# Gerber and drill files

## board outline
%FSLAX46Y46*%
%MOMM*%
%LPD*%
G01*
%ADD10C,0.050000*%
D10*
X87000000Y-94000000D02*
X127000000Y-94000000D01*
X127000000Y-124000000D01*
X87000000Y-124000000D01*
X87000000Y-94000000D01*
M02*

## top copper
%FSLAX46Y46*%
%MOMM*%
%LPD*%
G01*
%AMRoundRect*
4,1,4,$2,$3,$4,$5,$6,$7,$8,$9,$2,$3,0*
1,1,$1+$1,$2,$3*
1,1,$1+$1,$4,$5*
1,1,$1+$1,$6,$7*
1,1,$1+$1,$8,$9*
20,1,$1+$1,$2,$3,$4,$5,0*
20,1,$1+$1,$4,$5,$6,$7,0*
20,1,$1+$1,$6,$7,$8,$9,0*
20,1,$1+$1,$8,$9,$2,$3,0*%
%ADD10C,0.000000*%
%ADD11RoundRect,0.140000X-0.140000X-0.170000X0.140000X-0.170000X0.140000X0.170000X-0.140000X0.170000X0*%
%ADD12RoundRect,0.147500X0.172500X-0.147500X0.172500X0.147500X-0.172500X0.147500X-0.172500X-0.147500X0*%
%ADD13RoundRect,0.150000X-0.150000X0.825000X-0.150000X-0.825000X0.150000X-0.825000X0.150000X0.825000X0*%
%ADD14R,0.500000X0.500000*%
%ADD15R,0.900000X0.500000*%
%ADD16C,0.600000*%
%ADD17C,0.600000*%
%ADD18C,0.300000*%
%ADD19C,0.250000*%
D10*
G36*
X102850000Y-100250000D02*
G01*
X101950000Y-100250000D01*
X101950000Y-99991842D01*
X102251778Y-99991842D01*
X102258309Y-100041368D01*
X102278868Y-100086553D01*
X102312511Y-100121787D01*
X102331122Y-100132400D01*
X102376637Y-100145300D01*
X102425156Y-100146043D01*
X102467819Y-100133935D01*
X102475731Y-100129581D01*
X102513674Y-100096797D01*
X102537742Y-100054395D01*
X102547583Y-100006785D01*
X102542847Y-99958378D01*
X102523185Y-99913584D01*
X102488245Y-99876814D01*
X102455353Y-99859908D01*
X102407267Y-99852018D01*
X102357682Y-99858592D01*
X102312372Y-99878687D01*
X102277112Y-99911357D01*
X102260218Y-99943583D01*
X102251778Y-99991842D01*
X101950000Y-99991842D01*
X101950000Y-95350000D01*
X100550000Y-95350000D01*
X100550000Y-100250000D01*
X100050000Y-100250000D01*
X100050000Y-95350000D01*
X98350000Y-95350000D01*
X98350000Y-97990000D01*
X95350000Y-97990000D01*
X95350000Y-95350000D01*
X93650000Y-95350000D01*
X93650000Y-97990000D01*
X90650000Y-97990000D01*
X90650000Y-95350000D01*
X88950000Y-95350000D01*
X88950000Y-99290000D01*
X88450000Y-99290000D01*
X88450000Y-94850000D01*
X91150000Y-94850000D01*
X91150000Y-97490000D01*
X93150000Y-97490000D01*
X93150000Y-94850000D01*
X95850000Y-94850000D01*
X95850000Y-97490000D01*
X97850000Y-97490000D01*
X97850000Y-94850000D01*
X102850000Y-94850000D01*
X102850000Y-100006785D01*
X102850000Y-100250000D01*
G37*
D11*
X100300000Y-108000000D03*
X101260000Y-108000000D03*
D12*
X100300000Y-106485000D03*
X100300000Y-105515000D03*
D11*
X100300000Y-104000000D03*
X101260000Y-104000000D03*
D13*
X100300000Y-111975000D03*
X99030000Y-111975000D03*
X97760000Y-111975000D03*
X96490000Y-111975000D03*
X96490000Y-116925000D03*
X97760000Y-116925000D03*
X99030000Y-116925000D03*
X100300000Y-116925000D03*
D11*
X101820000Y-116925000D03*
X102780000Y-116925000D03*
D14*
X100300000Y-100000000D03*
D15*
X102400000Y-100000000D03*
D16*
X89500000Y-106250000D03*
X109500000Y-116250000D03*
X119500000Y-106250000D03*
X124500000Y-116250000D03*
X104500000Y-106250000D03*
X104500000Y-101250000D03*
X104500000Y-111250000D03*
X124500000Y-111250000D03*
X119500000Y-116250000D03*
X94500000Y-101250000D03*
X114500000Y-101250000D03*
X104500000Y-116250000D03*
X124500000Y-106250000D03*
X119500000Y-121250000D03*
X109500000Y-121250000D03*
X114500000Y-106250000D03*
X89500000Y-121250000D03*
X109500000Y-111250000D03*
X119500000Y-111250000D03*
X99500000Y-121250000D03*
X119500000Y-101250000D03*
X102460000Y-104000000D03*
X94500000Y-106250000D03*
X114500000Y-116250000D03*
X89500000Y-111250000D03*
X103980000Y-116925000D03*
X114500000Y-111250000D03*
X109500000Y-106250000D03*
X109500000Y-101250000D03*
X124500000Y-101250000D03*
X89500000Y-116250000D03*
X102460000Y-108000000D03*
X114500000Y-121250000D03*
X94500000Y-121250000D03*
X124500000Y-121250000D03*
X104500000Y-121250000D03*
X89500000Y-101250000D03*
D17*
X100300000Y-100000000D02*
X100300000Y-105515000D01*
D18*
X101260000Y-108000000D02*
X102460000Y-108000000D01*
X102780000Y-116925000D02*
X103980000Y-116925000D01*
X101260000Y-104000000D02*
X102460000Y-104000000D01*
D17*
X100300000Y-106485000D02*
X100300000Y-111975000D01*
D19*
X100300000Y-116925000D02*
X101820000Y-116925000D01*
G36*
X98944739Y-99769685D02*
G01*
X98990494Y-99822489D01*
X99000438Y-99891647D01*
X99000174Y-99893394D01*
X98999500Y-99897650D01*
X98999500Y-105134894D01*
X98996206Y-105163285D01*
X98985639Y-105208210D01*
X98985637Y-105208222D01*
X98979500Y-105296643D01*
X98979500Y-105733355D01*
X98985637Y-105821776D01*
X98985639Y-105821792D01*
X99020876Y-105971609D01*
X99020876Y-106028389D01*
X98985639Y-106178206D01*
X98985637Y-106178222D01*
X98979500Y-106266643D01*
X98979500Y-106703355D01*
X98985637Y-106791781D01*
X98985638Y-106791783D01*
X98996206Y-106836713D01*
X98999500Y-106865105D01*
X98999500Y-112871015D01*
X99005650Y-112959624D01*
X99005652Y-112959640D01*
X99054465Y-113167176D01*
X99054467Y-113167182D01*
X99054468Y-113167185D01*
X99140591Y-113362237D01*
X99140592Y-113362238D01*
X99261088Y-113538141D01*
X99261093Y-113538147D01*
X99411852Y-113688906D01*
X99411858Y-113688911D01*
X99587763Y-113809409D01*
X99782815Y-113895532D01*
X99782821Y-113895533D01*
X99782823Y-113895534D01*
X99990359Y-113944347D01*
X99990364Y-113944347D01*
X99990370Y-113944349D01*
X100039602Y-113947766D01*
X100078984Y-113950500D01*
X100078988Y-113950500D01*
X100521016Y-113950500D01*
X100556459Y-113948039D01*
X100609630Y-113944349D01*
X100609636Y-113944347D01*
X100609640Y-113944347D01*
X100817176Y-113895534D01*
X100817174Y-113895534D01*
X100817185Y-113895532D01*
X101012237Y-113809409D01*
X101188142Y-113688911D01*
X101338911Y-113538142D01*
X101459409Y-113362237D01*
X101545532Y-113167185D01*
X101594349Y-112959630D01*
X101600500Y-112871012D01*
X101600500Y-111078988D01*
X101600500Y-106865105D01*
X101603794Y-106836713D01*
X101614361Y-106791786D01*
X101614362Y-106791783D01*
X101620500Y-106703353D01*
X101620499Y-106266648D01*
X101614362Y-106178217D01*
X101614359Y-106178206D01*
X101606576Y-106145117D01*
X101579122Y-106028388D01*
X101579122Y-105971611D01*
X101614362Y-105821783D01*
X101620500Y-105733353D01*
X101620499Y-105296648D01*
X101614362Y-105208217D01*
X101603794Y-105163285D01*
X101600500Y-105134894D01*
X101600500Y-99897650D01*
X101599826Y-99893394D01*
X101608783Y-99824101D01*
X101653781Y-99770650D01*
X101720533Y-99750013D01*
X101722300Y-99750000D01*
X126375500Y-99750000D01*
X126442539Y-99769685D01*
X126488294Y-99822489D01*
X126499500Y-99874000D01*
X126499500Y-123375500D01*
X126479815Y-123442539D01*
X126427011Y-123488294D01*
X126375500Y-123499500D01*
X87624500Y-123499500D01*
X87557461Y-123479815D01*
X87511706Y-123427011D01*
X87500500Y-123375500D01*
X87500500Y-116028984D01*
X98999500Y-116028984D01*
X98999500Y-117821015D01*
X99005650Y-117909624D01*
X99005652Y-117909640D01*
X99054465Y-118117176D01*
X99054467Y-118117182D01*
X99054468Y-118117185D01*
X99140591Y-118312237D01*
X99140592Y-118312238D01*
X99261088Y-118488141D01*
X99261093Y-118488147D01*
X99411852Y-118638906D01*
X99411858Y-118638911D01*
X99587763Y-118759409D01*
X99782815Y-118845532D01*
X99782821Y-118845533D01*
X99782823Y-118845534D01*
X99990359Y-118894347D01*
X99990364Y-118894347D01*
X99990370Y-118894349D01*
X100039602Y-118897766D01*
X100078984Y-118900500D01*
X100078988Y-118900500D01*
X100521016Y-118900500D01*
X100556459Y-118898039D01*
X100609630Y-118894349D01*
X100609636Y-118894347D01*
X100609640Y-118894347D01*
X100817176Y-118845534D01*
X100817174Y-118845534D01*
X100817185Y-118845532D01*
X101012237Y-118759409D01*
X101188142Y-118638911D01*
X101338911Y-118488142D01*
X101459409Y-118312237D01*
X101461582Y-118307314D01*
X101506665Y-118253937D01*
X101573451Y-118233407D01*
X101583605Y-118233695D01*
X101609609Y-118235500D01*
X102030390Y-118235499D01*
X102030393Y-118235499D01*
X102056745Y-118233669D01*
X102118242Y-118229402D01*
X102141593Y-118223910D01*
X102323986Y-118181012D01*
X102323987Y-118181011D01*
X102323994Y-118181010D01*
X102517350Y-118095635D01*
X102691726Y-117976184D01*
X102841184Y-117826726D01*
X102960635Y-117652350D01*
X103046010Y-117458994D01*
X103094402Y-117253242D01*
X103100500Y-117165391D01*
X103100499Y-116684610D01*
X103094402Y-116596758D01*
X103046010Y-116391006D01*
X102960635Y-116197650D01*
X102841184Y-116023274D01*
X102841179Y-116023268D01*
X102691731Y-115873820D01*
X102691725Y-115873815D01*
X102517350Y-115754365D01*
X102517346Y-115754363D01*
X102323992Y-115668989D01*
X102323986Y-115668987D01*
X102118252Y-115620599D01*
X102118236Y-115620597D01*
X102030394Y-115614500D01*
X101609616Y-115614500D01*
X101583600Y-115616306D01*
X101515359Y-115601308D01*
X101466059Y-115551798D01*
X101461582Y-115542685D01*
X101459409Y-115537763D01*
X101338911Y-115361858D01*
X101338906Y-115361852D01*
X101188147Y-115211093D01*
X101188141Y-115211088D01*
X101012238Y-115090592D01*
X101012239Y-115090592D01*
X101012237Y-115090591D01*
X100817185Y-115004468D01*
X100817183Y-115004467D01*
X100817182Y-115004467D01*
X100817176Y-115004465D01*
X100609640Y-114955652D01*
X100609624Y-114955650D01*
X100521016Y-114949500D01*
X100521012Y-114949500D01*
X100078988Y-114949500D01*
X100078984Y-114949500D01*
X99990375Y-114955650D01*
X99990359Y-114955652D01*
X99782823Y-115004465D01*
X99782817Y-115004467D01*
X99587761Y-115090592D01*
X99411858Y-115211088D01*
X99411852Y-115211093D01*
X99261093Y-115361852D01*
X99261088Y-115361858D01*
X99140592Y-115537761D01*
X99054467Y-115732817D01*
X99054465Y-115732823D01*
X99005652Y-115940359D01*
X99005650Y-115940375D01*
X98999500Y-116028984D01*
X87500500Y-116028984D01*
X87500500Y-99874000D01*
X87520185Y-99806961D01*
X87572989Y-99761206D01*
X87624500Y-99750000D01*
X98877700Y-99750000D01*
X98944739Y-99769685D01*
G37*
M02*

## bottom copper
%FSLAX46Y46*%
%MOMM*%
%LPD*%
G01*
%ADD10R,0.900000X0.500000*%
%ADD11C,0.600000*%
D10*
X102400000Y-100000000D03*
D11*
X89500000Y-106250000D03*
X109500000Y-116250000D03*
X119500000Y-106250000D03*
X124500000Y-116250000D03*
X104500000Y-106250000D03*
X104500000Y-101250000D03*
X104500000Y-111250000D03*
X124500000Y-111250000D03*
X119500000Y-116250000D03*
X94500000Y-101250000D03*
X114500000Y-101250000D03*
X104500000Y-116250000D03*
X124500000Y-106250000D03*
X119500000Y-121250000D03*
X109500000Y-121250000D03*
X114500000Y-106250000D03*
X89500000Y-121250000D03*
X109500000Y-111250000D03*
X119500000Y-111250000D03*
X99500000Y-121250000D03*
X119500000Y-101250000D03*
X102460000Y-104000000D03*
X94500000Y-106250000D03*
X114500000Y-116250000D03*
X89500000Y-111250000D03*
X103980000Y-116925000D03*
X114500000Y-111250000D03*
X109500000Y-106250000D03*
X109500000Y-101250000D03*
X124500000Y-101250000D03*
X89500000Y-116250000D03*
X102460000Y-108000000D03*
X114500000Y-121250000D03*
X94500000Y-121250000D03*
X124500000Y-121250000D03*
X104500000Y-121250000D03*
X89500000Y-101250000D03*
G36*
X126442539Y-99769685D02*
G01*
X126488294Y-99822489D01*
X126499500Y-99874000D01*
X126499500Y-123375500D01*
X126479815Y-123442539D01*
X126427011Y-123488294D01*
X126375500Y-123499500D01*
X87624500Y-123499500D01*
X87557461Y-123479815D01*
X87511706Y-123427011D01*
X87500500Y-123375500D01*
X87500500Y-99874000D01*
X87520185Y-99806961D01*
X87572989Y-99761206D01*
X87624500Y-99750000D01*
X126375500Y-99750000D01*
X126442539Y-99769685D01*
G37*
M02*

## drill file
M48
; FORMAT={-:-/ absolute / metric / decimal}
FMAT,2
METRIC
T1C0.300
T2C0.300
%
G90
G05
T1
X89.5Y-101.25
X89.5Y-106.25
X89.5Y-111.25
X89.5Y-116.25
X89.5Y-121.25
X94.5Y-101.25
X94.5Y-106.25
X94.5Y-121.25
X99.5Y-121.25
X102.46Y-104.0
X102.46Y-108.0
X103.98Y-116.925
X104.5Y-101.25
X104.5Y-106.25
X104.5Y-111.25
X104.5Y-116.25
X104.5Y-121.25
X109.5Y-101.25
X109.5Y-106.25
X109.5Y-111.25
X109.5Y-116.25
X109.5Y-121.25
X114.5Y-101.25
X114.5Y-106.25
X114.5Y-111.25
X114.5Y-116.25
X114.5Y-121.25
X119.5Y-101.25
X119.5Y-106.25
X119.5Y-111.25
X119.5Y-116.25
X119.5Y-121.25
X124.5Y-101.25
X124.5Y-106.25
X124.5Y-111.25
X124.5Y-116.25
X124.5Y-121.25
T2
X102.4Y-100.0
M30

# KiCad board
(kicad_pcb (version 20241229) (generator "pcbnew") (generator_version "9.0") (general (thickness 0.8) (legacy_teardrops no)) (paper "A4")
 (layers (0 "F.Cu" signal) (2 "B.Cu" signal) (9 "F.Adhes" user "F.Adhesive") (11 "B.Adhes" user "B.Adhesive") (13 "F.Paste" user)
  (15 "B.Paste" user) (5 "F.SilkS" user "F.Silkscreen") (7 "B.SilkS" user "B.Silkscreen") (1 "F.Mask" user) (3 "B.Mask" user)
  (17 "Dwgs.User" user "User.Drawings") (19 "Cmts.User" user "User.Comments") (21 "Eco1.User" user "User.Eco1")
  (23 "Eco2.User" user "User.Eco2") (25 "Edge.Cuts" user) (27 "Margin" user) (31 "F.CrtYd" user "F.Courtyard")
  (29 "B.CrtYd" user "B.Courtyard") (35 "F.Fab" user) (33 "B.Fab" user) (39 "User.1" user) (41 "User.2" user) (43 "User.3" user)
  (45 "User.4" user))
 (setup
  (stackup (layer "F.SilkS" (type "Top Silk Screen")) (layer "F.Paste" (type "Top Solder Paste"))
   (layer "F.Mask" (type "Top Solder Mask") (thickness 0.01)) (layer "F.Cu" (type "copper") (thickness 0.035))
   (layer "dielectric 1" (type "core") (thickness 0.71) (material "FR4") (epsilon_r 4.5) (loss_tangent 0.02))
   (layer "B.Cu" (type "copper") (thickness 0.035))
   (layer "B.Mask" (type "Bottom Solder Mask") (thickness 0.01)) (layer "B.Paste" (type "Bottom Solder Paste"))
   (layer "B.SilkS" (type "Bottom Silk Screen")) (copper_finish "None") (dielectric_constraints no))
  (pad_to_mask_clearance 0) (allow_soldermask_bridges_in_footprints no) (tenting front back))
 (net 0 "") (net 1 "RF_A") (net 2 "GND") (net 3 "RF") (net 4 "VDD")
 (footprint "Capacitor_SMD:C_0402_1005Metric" (layer "F.Cu") (at 100.78 108)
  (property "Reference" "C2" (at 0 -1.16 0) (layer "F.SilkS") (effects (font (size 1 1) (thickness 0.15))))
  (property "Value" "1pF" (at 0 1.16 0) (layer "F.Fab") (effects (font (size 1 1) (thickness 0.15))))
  (pad "1" smd roundrect (at -0.48 0) (size 0.56 0.62) (layers "F.Cu" "F.Mask" "F.Paste") (roundrect_rratio 0.25) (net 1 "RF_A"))
  (pad "2" smd roundrect (at 0.48 0) (size 0.56 0.62) (layers "F.Cu" "F.Mask" "F.Paste") (roundrect_rratio 0.25) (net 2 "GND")))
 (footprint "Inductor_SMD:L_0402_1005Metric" (layer "F.Cu") (at 100.3 106 90)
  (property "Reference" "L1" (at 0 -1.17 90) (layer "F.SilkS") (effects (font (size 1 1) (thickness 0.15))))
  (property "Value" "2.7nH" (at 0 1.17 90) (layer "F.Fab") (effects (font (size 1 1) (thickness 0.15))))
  (pad "1" smd roundrect (at -0.485 0 90) (size 0.59 0.64) (layers "F.Cu" "F.Mask" "F.Paste") (roundrect_rratio 0.25) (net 1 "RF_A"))
  (pad "2" smd roundrect (at 0.485 0 90) (size 0.59 0.64) (layers "F.Cu" "F.Mask" "F.Paste") (roundrect_rratio 0.25) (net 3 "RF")))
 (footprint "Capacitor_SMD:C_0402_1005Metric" (layer "F.Cu") (at 100.78 104)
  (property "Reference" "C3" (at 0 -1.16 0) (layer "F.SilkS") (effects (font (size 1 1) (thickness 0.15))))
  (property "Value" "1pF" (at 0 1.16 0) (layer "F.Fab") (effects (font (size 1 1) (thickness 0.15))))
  (pad "1" smd roundrect (at -0.48 0) (size 0.56 0.62) (layers "F.Cu" "F.Mask" "F.Paste") (roundrect_rratio 0.25) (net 3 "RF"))
  (pad "2" smd roundrect (at 0.48 0) (size 0.56 0.62) (layers "F.Cu" "F.Mask" "F.Paste") (roundrect_rratio 0.25) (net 2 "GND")))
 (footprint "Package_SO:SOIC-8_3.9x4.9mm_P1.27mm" (layer "F.Cu") (at 98.395 114.45 -90)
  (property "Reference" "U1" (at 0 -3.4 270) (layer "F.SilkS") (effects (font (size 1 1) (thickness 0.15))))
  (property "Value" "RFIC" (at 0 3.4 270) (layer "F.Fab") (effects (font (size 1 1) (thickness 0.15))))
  (pad "1" smd roundrect (at -2.475 -1.905 270) (size 1.95 0.6) (layers "F.Cu" "F.Mask" "F.Paste") (roundrect_rratio 0.25) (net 1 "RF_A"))
  (pad "2" smd roundrect (at -2.475 -0.635 270) (size 1.95 0.6) (layers "F.Cu" "F.Mask" "F.Paste") (roundrect_rratio 0.25) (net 2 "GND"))
  (pad "3" smd roundrect (at -2.475 0.635 270) (size 1.95 0.6) (layers "F.Cu" "F.Mask" "F.Paste") (roundrect_rratio 0.25) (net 2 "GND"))
  (pad "4" smd roundrect (at -2.475 1.905 270) (size 1.95 0.6) (layers "F.Cu" "F.Mask" "F.Paste") (roundrect_rratio 0.25) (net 2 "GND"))
  (pad "5" smd roundrect (at 2.475 1.905 270) (size 1.95 0.6) (layers "F.Cu" "F.Mask" "F.Paste") (roundrect_rratio 0.25) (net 2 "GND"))
  (pad "6" smd roundrect (at 2.475 0.635 270) (size 1.95 0.6) (layers "F.Cu" "F.Mask" "F.Paste") (roundrect_rratio 0.25) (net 2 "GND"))
  (pad "7" smd roundrect (at 2.475 -0.635 270) (size 1.95 0.6) (layers "F.Cu" "F.Mask" "F.Paste") (roundrect_rratio 0.25) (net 2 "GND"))
  (pad "8" smd roundrect (at 2.475 -1.905 270) (size 1.95 0.6) (layers "F.Cu" "F.Mask" "F.Paste") (roundrect_rratio 0.25) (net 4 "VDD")))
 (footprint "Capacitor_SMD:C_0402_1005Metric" (layer "F.Cu") (at 102.3 116.925)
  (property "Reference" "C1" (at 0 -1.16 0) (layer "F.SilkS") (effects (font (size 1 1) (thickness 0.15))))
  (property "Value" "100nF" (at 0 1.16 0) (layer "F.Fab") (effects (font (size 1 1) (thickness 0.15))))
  (pad "1" smd roundrect (at -0.48 0) (size 0.56 0.62) (layers "F.Cu" "F.Mask" "F.Paste") (roundrect_rratio 0.25) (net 4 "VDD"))
  (pad "2" smd roundrect (at 0.48 0) (size 0.56 0.62) (layers "F.Cu" "F.Mask" "F.Paste") (roundrect_rratio 0.25) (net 2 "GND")))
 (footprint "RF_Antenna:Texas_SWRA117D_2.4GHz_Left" (layer "F.Cu") (at 100.3 100)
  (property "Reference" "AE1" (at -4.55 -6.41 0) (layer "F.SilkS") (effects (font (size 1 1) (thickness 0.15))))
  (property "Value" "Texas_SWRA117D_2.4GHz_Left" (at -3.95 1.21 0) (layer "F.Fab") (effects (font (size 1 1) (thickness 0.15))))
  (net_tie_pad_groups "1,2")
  (fp_poly
   (pts (xy -2.45 -2.51) (xy -4.45 -2.51) (xy -4.45 -5.15) (xy -7.15 -5.15) (xy -7.15 -2.51) (xy -9.15 -2.51) (xy -9.15 -5.15)
    (xy -11.85 -5.15) (xy -11.85 -0.71) (xy -11.35 -0.71) (xy -11.35 -4.65) (xy -9.65 -4.65) (xy -9.65 -2.01) (xy -6.65 -2.01)
    (xy -6.65 -4.65) (xy -4.95 -4.65) (xy -4.95 -2.01) (xy -1.95 -2.01) (xy -1.95 -4.65) (xy -0.25 -4.65) (xy -0.25 0.25) (xy 0.25 0.25)
    (xy 0.25 -4.65) (xy 1.65 -4.65) (xy 1.65 0.25) (xy 2.55 0.25) (xy 2.55 0.006785) (xy 2.247583 0.006785) (xy 2.237742 0.054395)
    (xy 2.213674 0.096797) (xy 2.175731 0.129581) (xy 2.167819 0.133935) (xy 2.125156 0.146043) (xy 2.076637 0.1453) (xy 2.031122 0.1324)
    (xy 2.012511 0.121787) (xy 1.978868 0.086553) (xy 1.958309 0.041368) (xy 1.951778 -0.008158) (xy 1.960218 -0.056417)
    (xy 1.977112 -0.088643) (xy 2.012372 -0.121313) (xy 2.057682 -0.141408) (xy 2.107267 -0.147982) (xy 2.155353 -0.140092)
    (xy 2.188245 -0.123186) (xy 2.223185 -0.086416) (xy 2.242847 -0.041622) (xy 2.247583 0.006785) (xy 2.55 0.006785) (xy 2.55 -5.15)
    (xy -2.45 -5.15) (xy -2.45 -2.51))
   (stroke (width 0) (type solid)) (fill yes) (layer "F.Cu"))
  (pad "1" connect rect (at 0 0) (size 0.5 0.5) (layers "F.Cu") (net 3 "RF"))
  (pad "2" thru_hole rect (at 2.1 0) (size 0.9 0.5) (drill 0.3) (layers "*.Cu") (remove_unused_layers no) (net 2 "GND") (zone_connect 2)))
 (gr_rect (start 87 94) (end 127 124) (stroke (width 0.05) (type default)) (fill no) (layer "Edge.Cuts"))
 (segment (start 100.3 100) (end 100.3 105.515) (width 0.6) (layer "F.Cu") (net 3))
 (segment (start 101.26 108) (end 102.46 108) (width 0.3) (layer "F.Cu") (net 2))
 (segment (start 102.78 116.925) (end 103.98 116.925) (width 0.3) (layer "F.Cu") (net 2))
 (segment (start 101.26 104) (end 102.46 104) (width 0.3) (layer "F.Cu") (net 2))
 (via (at 89.5 106.25) (size 0.6) (drill 0.3) (layers "F.Cu" "B.Cu") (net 2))
 (via (at 109.5 116.25) (size 0.6) (drill 0.3) (layers "F.Cu" "B.Cu") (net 2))
 (via (at 119.5 106.25) (size 0.6) (drill 0.3) (layers "F.Cu" "B.Cu") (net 2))
 (via (at 124.5 116.25) (size 0.6) (drill 0.3) (layers "F.Cu" "B.Cu") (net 2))
 (via (at 104.5 106.25) (size 0.6) (drill 0.3) (layers "F.Cu" "B.Cu") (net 2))
 (via (at 104.5 101.25) (size 0.6) (drill 0.3) (layers "F.Cu" "B.Cu") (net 2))
 (via (at 104.5 111.25) (size 0.6) (drill 0.3) (layers "F.Cu" "B.Cu") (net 2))
 (via (at 124.5 111.25) (size 0.6) (drill 0.3) (layers "F.Cu" "B.Cu") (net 2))
 (via (at 119.5 116.25) (size 0.6) (drill 0.3) (layers "F.Cu" "B.Cu") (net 2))
 (via (at 94.5 101.25) (size 0.6) (drill 0.3) (layers "F.Cu" "B.Cu") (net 2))
 (via (at 114.5 101.25) (size 0.6) (drill 0.3) (layers "F.Cu" "B.Cu") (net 2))
 (via (at 104.5 116.25) (size 0.6) (drill 0.3) (layers "F.Cu" "B.Cu") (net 2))
 (via (at 124.5 106.25) (size 0.6) (drill 0.3) (layers "F.Cu" "B.Cu") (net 2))
 (via (at 119.5 121.25) (size 0.6) (drill 0.3) (layers "F.Cu" "B.Cu") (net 2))
 (via (at 109.5 121.25) (size 0.6) (drill 0.3) (layers "F.Cu" "B.Cu") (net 2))
 (via (at 114.5 106.25) (size 0.6) (drill 0.3) (layers "F.Cu" "B.Cu") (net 2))
 (via (at 89.5 121.25) (size 0.6) (drill 0.3) (layers "F.Cu" "B.Cu") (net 2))
 (via (at 109.5 111.25) (size 0.6) (drill 0.3) (layers "F.Cu" "B.Cu") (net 2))
 (via (at 119.5 111.25) (size 0.6) (drill 0.3) (layers "F.Cu" "B.Cu") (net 2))
 (via (at 99.5 121.25) (size 0.6) (drill 0.3) (layers "F.Cu" "B.Cu") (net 2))
 (via (at 119.5 101.25) (size 0.6) (drill 0.3) (layers "F.Cu" "B.Cu") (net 2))
 (via (at 102.46 104) (size 0.6) (drill 0.3) (layers "F.Cu" "B.Cu") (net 2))
 (via (at 94.5 106.25) (size 0.6) (drill 0.3) (layers "F.Cu" "B.Cu") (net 2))
 (via (at 114.5 116.25) (size 0.6) (drill 0.3) (layers "F.Cu" "B.Cu") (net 2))
 (via (at 89.5 111.25) (size 0.6) (drill 0.3) (layers "F.Cu" "B.Cu") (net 2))
 (via (at 103.98 116.925) (size 0.6) (drill 0.3) (layers "F.Cu" "B.Cu") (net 2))
 (via (at 114.5 111.25) (size 0.6) (drill 0.3) (layers "F.Cu" "B.Cu") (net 2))
 (via (at 109.5 106.25) (size 0.6) (drill 0.3) (layers "F.Cu" "B.Cu") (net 2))
 (via (at 109.5 101.25) (size 0.6) (drill 0.3) (layers "F.Cu" "B.Cu") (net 2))
 (via (at 124.5 101.25) (size 0.6) (drill 0.3) (layers "F.Cu" "B.Cu") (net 2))
 (via (at 89.5 116.25) (size 0.6) (drill 0.3) (layers "F.Cu" "B.Cu") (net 2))
 (via (at 102.46 108) (size 0.6) (drill 0.3) (layers "F.Cu" "B.Cu") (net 2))
 (via (at 114.5 121.25) (size 0.6) (drill 0.3) (layers "F.Cu" "B.Cu") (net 2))
 (via (at 94.5 121.25) (size 0.6) (drill 0.3) (layers "F.Cu" "B.Cu") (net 2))
 (via (at 124.5 121.25) (size 0.6) (drill 0.3) (layers "F.Cu" "B.Cu") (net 2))
 (via (at 104.5 121.25) (size 0.6) (drill 0.3) (layers "F.Cu" "B.Cu") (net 2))
 (via (at 89.5 101.25) (size 0.6) (drill 0.3) (layers "F.Cu" "B.Cu") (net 2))
 (segment (start 100.3 106.485) (end 100.3 111.975) (width 0.6) (layer "F.Cu") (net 1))
 (segment (start 100.3 116.925) (end 101.82 116.925) (width 0.25) (layer "F.Cu") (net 4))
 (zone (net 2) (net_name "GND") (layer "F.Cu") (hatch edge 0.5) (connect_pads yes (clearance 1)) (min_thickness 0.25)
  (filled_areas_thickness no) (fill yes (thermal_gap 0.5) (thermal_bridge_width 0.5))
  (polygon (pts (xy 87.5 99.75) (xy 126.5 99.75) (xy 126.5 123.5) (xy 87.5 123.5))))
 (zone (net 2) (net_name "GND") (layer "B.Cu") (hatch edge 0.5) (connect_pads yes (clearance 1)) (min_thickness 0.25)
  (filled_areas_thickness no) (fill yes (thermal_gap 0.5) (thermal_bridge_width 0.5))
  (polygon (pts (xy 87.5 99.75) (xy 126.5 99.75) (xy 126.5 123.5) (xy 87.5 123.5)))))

